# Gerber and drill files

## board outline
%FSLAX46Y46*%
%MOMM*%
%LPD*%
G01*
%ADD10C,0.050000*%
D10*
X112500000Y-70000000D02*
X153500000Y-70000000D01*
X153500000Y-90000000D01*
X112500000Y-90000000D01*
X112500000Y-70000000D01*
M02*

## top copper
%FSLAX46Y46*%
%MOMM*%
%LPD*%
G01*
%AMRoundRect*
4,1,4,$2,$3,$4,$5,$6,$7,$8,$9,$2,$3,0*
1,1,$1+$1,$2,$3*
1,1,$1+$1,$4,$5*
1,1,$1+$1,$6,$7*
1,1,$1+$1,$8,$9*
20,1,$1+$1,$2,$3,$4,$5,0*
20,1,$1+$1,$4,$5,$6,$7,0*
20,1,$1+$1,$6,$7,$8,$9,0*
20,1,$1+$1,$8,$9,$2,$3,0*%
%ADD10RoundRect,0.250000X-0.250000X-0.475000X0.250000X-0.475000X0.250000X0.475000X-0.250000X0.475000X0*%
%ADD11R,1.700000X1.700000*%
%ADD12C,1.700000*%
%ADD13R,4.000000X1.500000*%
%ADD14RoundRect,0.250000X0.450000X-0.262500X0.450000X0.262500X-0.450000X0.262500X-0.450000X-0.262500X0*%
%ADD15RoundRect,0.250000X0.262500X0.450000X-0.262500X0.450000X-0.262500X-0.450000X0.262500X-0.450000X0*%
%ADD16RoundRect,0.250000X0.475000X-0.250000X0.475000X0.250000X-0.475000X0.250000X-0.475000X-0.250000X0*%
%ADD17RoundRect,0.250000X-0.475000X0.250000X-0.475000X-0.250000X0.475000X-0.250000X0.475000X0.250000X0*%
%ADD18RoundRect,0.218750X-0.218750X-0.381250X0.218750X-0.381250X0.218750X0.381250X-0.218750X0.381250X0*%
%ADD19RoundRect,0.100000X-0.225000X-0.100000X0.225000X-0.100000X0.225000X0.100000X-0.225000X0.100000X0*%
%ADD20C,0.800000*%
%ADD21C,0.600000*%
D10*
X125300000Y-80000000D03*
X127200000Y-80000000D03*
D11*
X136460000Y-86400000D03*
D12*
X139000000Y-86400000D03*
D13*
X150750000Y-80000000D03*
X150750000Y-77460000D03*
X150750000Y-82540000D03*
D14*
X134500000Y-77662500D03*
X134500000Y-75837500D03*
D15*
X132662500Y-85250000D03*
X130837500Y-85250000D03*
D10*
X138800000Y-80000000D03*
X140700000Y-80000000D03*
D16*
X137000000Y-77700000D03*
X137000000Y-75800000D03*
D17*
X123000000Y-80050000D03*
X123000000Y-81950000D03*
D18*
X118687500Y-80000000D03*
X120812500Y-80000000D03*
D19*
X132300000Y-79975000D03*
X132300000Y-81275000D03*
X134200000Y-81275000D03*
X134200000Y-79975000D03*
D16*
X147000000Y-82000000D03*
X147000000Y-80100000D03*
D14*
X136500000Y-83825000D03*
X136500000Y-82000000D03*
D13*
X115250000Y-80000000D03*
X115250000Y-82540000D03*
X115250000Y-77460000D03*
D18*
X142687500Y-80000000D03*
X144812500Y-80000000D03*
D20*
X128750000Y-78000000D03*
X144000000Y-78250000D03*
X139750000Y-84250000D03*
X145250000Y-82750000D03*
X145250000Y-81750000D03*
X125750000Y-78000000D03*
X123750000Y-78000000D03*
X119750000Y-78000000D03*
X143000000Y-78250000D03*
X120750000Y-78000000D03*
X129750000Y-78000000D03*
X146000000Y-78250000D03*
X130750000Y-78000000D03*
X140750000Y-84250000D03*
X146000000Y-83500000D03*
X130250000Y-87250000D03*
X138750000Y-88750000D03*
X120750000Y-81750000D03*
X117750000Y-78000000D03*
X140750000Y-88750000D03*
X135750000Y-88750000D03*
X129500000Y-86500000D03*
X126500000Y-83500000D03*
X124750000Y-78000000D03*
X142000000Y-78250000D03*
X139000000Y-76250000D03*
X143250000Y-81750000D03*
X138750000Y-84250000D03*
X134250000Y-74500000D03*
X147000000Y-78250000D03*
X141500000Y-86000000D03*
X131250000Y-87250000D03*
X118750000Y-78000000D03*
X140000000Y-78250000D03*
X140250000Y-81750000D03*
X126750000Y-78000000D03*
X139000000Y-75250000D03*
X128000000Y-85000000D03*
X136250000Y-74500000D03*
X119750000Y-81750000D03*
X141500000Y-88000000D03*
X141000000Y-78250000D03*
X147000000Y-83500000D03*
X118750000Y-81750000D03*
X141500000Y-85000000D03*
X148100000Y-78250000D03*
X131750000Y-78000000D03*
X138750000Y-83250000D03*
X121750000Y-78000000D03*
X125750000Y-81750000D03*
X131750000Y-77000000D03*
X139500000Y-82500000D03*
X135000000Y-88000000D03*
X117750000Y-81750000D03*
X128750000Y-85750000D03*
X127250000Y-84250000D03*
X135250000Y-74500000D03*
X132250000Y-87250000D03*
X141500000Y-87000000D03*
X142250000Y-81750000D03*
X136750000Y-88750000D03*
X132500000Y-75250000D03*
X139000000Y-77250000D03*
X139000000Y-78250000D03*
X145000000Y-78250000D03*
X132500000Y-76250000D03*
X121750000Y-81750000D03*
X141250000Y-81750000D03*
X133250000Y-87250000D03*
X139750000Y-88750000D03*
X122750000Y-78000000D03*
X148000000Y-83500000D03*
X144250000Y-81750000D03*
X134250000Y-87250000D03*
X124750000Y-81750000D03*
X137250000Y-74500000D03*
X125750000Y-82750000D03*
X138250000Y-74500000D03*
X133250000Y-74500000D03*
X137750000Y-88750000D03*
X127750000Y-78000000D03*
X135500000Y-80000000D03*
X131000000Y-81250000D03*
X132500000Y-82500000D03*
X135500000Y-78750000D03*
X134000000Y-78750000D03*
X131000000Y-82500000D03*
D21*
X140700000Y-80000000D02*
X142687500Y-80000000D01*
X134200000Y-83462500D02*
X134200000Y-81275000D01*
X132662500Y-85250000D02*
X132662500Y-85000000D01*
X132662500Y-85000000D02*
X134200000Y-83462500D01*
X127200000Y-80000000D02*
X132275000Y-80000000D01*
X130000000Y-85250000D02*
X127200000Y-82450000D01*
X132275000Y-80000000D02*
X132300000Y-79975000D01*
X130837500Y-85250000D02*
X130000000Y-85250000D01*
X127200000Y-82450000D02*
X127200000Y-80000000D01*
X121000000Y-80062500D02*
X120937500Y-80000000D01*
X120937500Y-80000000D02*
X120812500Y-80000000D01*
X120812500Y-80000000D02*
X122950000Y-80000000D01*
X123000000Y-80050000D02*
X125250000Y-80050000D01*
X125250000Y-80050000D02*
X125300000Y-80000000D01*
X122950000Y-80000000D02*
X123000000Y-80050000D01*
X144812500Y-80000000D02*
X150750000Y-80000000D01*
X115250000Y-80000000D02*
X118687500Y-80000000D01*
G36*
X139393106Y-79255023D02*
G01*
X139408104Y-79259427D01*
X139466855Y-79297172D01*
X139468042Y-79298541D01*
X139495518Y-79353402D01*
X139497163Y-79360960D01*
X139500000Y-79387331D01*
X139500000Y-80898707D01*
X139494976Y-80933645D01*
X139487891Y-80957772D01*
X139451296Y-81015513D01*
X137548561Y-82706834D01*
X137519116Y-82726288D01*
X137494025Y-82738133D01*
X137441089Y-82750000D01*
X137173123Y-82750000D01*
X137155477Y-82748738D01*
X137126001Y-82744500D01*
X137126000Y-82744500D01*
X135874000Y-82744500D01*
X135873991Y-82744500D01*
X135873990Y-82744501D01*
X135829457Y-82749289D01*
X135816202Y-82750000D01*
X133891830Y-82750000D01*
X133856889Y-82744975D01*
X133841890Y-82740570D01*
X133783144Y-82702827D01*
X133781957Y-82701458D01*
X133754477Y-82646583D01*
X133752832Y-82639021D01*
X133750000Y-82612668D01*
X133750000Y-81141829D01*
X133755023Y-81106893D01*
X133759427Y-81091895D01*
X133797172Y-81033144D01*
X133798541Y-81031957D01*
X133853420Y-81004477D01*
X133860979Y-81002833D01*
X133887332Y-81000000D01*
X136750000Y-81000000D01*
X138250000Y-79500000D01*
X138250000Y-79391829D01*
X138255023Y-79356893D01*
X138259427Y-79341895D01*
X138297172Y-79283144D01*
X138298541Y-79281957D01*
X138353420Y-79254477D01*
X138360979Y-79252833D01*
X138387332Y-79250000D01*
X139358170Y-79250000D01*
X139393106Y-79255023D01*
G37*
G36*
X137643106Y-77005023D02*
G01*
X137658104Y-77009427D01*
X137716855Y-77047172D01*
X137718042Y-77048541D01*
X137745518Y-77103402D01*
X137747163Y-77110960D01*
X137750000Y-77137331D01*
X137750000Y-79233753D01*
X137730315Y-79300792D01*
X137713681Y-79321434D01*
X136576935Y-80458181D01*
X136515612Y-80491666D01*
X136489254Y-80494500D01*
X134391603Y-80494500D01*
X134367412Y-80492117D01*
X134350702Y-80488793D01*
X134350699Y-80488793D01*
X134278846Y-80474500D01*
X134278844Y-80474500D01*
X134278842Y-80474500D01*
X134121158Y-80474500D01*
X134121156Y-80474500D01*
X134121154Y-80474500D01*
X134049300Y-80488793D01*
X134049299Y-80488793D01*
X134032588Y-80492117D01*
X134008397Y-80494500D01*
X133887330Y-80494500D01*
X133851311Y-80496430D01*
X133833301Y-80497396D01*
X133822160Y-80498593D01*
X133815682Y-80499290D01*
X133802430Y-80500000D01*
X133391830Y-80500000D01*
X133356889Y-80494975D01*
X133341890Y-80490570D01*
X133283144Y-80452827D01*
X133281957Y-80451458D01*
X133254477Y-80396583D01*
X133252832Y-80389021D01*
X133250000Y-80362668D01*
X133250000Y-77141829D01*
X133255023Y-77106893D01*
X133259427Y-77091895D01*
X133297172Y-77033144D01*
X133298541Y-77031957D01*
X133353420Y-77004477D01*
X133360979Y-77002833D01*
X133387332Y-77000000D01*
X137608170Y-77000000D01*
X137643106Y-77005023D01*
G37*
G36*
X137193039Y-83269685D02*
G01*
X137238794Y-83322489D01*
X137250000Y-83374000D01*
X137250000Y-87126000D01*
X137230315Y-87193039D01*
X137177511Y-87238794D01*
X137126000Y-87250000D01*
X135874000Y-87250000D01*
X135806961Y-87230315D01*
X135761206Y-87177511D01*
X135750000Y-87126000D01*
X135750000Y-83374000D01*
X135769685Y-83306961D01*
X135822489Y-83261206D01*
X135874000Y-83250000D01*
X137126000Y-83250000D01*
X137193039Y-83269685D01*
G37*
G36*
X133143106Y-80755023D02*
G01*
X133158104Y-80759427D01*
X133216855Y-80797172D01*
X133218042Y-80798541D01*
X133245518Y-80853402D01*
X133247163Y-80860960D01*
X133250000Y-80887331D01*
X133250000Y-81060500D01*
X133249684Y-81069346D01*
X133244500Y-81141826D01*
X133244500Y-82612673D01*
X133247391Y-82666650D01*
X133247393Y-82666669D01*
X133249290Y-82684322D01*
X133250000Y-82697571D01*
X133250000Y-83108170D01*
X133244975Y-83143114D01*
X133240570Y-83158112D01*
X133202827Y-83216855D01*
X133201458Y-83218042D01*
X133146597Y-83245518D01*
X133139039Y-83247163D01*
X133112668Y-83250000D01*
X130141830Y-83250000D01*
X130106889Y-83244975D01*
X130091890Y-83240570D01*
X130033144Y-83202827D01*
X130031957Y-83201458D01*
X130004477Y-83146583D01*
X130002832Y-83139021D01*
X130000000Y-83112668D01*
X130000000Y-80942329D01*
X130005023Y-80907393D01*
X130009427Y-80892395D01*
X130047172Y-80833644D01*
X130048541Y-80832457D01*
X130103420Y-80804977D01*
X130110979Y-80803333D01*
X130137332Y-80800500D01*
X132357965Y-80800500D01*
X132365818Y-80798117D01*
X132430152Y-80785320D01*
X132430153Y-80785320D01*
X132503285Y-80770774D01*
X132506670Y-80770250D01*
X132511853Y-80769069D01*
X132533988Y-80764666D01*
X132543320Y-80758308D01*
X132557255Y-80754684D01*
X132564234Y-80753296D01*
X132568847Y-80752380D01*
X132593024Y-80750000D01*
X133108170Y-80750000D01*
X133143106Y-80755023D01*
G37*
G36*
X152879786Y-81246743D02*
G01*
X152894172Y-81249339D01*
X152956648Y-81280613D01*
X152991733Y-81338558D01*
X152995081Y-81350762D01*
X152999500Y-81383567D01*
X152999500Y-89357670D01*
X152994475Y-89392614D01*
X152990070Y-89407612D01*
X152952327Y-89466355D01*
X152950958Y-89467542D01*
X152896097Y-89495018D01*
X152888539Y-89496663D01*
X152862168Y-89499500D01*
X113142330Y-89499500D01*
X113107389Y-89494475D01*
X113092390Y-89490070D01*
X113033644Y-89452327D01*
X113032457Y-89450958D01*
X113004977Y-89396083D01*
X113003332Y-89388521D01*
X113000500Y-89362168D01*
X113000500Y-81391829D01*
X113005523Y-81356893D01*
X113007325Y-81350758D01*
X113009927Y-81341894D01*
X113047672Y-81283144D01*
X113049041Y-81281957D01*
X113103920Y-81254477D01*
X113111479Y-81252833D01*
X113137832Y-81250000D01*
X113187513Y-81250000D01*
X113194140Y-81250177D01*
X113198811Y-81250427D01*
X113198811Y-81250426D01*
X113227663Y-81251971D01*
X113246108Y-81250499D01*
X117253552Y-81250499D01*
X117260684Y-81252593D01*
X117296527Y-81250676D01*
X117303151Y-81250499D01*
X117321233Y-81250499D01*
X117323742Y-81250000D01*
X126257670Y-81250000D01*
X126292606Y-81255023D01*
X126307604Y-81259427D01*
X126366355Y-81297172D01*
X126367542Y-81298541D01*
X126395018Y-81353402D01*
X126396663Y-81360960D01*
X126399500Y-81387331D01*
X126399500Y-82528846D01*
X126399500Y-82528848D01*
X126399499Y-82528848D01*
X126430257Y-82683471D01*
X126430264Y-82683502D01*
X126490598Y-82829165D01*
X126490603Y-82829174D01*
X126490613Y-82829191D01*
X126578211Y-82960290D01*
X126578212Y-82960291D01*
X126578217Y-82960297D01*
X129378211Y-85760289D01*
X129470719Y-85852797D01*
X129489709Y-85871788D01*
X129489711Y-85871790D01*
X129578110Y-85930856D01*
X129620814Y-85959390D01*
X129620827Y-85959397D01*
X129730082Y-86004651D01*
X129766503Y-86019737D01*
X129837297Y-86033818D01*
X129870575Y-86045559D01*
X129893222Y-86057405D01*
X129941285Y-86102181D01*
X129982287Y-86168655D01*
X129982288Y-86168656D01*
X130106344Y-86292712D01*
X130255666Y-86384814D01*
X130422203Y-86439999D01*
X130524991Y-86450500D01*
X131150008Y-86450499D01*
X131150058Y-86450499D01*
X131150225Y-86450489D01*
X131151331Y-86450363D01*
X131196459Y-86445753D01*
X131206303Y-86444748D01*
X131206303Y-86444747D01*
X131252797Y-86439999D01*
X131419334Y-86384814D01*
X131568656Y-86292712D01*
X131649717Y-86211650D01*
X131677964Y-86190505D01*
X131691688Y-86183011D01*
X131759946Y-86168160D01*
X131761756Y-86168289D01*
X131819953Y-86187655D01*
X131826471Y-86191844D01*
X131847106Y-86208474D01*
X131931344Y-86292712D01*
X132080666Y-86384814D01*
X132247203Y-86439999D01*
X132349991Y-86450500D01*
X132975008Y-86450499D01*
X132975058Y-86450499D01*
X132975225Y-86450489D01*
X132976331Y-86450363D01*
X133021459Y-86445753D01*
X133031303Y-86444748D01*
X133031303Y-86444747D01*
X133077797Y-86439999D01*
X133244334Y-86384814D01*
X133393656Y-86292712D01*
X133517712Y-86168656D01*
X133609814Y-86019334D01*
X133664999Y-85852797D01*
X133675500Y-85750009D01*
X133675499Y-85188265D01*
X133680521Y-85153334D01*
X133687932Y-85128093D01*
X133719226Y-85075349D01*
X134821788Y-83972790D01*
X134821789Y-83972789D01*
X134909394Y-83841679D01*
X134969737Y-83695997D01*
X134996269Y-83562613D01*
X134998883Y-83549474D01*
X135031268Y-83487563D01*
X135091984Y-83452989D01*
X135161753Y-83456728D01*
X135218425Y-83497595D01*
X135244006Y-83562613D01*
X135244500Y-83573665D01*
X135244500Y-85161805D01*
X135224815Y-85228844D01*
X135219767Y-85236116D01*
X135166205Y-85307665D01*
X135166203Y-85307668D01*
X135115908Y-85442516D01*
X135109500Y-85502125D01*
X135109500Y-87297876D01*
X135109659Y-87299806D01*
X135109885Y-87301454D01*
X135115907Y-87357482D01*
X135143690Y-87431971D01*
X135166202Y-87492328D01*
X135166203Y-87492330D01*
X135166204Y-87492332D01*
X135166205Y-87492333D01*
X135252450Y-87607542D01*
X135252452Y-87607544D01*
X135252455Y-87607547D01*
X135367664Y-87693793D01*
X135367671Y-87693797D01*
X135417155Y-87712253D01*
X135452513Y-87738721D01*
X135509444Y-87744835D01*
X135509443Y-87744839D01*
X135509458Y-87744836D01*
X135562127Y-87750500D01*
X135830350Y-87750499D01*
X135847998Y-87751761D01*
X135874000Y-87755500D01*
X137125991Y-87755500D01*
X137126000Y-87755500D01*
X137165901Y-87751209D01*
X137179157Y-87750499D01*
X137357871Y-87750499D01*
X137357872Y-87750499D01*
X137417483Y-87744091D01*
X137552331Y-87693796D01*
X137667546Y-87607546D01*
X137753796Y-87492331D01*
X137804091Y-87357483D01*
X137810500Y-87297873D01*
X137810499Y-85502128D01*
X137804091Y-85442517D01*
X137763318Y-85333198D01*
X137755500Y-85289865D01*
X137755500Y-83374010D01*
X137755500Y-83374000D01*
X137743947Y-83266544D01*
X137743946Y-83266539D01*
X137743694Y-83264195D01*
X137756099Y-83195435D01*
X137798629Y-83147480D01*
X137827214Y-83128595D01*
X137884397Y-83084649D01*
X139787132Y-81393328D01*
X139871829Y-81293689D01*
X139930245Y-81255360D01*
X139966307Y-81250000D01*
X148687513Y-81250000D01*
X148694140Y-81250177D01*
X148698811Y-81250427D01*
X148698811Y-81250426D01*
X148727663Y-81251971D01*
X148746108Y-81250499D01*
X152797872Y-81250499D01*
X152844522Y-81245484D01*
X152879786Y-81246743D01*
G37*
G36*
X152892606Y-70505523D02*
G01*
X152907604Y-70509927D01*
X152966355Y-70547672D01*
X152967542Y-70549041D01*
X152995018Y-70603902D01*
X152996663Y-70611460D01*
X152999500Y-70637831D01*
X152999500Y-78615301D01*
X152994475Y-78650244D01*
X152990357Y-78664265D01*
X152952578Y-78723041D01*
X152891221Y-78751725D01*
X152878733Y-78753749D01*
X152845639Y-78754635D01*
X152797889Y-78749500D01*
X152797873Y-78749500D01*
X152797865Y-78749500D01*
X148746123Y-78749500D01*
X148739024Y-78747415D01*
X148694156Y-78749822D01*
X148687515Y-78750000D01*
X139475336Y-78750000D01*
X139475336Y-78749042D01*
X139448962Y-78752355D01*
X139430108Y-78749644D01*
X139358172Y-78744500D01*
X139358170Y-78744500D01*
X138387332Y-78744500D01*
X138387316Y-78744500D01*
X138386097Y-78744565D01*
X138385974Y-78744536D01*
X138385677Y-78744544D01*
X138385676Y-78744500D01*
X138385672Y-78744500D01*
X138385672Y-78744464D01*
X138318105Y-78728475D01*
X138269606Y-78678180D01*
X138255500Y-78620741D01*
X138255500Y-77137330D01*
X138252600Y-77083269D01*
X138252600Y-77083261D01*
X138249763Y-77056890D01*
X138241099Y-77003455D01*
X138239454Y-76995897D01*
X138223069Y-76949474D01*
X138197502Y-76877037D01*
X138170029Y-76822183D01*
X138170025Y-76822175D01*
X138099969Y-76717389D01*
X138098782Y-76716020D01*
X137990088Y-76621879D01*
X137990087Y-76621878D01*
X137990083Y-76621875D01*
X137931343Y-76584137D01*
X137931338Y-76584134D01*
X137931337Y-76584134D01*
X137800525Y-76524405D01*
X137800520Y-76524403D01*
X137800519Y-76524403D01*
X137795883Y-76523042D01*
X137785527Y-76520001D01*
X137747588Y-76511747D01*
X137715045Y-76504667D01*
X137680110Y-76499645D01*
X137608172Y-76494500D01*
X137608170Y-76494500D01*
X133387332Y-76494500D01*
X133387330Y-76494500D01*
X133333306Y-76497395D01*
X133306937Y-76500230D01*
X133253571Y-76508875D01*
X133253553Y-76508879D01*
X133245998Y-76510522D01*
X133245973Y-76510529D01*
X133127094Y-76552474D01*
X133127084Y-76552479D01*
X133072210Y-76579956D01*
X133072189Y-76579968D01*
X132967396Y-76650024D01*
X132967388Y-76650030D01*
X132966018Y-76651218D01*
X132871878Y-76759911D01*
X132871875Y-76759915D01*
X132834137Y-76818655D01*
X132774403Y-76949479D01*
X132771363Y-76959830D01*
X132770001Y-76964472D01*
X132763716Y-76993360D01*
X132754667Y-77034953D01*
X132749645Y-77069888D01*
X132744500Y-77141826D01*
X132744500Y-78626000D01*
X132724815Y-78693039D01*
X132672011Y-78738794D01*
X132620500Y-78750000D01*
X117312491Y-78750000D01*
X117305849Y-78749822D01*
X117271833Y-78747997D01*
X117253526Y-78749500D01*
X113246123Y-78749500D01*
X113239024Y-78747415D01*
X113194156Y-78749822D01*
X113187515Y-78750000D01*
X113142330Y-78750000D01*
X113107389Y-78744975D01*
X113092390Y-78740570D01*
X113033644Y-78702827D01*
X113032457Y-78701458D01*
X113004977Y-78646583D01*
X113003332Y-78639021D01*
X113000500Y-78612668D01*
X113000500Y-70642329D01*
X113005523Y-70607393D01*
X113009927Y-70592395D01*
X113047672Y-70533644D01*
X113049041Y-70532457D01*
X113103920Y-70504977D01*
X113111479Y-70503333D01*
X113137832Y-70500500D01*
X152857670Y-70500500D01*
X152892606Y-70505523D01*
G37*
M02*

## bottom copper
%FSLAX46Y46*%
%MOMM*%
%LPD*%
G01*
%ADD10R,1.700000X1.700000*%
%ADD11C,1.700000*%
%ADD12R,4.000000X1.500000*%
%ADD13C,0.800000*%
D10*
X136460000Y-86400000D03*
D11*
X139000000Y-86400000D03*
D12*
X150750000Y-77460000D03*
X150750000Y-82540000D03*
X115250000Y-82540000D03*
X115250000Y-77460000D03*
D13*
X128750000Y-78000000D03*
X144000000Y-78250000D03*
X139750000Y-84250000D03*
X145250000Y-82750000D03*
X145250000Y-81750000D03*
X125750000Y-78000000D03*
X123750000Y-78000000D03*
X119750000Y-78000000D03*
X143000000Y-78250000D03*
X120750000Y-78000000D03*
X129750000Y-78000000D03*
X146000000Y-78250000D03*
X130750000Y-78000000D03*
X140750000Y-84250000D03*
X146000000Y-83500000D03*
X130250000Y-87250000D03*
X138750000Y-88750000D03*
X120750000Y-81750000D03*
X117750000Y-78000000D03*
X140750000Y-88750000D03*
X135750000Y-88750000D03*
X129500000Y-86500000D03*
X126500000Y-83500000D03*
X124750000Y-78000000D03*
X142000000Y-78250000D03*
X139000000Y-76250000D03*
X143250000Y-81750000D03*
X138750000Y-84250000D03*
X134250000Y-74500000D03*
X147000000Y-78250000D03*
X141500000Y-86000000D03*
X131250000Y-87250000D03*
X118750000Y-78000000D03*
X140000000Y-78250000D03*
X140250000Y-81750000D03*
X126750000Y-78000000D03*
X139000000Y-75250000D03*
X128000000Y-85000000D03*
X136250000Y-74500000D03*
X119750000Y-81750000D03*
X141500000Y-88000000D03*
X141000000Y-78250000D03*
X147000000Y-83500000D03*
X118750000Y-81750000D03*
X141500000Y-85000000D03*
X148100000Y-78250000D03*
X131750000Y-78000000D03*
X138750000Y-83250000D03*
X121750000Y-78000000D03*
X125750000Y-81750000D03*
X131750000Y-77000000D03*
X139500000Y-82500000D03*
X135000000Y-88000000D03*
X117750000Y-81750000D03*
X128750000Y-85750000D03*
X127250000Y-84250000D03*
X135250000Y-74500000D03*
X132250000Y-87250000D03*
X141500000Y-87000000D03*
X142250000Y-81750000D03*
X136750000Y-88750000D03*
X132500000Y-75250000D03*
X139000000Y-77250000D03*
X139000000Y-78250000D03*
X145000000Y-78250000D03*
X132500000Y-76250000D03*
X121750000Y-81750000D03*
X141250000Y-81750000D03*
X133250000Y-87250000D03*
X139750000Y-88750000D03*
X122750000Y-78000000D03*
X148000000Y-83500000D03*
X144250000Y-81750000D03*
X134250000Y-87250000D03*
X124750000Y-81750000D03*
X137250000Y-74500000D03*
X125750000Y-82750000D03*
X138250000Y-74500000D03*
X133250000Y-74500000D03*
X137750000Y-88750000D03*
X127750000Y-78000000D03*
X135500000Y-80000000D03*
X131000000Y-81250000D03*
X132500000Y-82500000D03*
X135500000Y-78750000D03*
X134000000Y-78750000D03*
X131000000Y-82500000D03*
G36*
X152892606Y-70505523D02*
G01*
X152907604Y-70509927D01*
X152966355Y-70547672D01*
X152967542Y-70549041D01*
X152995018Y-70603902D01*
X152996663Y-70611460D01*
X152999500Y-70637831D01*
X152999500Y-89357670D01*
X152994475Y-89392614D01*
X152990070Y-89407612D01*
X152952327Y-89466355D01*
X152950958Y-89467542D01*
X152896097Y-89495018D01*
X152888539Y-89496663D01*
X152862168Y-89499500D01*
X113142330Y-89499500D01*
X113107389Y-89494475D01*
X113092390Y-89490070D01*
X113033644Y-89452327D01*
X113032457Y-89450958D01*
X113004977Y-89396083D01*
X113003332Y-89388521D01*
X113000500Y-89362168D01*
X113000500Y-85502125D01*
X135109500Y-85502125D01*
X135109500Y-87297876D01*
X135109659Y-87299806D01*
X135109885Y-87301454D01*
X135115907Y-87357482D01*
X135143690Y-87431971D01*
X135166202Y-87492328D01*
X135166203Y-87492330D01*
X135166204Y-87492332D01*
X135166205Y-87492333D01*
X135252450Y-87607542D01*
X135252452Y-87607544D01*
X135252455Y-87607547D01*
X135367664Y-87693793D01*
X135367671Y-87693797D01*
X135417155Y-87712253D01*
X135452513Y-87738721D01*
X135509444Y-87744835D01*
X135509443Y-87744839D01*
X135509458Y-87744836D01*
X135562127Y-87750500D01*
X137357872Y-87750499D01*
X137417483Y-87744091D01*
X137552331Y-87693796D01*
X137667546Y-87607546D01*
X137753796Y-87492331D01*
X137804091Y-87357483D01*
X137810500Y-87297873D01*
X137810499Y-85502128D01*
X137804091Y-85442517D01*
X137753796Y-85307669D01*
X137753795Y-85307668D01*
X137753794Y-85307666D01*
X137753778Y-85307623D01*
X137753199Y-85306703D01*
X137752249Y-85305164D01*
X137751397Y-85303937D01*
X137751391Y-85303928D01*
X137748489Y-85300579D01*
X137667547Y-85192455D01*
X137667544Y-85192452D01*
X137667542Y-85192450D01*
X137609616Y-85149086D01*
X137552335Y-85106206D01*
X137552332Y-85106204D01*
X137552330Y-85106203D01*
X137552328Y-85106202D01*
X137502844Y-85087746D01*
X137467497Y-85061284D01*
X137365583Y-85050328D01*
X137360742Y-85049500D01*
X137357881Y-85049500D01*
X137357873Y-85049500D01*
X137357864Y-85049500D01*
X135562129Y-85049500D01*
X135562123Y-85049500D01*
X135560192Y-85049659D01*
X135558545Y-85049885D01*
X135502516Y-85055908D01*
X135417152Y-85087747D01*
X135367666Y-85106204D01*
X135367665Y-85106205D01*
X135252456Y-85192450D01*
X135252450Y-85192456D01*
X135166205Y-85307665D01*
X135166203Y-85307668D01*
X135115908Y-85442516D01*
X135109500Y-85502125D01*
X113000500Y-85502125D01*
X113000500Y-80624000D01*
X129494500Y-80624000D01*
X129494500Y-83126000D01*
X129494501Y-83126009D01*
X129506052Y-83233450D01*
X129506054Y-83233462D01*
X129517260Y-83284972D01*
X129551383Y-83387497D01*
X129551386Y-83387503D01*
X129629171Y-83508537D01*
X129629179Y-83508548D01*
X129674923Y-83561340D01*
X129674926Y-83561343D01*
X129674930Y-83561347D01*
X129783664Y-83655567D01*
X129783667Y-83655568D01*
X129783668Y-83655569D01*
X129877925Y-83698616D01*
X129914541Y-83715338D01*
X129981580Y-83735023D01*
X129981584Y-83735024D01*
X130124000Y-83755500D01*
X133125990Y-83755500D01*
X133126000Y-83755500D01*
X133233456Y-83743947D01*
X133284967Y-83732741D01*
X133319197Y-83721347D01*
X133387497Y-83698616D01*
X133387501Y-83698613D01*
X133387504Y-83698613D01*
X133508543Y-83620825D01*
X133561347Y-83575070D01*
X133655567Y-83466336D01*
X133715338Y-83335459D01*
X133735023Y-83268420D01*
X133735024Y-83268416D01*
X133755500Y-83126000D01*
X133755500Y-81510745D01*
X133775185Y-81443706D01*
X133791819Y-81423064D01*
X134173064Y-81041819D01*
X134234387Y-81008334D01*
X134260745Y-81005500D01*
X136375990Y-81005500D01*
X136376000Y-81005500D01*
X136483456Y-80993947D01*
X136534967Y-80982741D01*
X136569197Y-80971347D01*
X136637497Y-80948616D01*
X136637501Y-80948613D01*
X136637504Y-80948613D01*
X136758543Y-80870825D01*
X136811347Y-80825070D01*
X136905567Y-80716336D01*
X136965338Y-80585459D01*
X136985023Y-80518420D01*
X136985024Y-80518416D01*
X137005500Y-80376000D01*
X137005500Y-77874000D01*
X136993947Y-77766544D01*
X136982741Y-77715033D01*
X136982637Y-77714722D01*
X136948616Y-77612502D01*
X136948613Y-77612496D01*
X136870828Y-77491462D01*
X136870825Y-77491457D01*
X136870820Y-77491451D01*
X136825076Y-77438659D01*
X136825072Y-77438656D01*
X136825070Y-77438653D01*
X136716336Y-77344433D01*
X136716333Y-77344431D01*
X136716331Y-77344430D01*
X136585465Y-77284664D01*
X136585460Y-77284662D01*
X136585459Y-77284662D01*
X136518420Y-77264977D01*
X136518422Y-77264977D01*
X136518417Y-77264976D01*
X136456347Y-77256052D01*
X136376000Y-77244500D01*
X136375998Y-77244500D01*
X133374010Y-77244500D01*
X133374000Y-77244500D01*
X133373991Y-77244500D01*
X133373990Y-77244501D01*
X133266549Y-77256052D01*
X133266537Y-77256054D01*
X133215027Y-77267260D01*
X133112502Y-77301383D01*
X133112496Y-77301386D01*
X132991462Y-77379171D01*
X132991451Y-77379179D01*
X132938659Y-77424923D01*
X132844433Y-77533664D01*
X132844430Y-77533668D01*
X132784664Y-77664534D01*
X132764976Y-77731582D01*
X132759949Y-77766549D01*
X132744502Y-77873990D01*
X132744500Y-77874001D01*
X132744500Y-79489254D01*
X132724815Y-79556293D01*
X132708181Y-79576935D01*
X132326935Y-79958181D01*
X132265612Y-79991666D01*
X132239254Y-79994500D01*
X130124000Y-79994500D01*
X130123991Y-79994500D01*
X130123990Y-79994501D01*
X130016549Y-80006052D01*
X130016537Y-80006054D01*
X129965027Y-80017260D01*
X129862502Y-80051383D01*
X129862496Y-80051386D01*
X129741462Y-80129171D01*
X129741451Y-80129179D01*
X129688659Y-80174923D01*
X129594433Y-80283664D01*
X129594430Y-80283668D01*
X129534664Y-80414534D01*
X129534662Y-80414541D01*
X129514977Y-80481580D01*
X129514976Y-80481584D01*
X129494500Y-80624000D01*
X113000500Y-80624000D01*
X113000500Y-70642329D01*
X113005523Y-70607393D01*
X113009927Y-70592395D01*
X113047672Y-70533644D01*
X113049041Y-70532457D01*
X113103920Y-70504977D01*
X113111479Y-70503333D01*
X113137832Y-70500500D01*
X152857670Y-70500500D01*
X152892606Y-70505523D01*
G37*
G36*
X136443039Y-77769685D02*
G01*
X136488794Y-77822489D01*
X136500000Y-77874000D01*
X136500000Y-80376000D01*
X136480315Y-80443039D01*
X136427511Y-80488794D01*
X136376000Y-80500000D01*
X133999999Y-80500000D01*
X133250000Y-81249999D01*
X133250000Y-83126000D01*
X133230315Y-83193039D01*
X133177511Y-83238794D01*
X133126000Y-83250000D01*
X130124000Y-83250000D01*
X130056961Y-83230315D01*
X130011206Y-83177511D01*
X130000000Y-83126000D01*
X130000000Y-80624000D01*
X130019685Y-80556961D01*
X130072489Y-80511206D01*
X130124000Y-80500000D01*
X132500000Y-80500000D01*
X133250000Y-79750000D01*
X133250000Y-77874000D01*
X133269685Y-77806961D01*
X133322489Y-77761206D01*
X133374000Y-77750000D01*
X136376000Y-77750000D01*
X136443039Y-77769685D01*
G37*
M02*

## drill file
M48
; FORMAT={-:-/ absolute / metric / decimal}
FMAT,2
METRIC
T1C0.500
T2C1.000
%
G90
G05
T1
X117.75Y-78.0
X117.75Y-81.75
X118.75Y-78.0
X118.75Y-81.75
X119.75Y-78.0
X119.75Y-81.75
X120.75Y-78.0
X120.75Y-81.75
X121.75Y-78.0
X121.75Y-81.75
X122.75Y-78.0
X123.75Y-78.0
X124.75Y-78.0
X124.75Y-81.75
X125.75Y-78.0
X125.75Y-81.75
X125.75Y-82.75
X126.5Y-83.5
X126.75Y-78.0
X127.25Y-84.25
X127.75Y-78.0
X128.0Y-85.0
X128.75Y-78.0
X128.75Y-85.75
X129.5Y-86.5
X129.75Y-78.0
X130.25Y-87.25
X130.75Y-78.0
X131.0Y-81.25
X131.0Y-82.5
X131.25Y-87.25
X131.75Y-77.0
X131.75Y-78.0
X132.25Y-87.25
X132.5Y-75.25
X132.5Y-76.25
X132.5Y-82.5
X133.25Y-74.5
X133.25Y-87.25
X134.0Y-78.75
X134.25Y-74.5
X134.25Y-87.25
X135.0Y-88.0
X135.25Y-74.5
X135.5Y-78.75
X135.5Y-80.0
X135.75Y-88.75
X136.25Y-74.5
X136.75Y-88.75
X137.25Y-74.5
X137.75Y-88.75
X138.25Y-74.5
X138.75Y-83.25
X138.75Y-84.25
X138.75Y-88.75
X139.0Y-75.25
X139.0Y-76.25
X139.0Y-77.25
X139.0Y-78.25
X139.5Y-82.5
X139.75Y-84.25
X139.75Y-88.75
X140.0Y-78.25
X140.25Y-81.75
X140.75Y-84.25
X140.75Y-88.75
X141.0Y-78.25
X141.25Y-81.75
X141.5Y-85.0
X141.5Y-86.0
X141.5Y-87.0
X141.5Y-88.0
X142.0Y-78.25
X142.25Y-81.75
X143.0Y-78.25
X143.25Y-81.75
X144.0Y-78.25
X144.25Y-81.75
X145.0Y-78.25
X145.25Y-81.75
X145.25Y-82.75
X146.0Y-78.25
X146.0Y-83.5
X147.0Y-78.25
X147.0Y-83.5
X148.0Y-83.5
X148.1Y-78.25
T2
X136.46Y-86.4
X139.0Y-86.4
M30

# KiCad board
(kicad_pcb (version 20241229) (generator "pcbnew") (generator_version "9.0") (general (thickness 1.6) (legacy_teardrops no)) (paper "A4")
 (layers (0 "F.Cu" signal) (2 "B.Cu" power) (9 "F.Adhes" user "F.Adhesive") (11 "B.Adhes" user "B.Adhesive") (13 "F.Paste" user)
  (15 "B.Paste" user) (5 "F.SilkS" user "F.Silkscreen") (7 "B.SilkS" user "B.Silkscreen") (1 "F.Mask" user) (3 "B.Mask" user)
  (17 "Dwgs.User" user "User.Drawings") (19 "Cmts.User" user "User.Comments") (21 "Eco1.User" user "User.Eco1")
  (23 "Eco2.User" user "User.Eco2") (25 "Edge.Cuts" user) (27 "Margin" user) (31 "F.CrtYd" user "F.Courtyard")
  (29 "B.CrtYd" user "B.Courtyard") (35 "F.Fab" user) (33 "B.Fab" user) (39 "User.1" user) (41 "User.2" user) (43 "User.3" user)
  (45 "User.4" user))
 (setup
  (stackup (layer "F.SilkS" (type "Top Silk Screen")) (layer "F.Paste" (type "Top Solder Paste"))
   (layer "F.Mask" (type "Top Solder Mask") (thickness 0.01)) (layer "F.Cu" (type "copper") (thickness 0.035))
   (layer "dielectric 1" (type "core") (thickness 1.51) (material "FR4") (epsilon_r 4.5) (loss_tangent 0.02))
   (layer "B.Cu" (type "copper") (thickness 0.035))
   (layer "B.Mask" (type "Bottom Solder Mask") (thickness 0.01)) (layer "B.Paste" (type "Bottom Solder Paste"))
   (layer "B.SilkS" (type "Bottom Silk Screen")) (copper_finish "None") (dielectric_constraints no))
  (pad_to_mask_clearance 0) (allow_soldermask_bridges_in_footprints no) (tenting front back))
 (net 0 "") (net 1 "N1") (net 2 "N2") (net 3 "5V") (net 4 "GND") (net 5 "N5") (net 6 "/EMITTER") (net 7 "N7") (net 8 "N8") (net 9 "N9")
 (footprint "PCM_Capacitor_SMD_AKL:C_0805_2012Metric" (layer "F.Cu") (at 126.25 80)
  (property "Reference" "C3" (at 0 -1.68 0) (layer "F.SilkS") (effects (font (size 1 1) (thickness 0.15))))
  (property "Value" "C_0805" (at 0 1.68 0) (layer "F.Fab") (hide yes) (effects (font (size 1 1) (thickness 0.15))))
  (pad "1" smd roundrect (at -0.95 0) (size 1 1.45) (layers "F.Cu" "F.Mask" "F.Paste") (roundrect_rratio 0.25) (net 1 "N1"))
  (pad "2" smd roundrect (at 0.95 0) (size 1 1.45) (layers "F.Cu" "F.Mask" "F.Paste") (roundrect_rratio 0.25) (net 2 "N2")))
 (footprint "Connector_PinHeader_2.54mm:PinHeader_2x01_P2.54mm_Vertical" (layer "F.Cu") (at 136.46 86.4)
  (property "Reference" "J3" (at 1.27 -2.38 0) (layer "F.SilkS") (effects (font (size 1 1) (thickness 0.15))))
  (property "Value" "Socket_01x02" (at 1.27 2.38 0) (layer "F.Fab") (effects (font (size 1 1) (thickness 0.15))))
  (pad "1" thru_hole rect (at 0 0) (size 1.7 1.7) (drill 1) (layers "*.Cu" "*.Mask") (remove_unused_layers no) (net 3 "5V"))
  (pad "2" thru_hole circle (at 2.54 0) (size 1.7 1.7) (drill 1) (layers "*.Cu" "*.Mask") (remove_unused_layers no) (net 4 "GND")))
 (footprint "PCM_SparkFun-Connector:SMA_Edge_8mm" (layer "F.Cu") (at 150.75 80 -90)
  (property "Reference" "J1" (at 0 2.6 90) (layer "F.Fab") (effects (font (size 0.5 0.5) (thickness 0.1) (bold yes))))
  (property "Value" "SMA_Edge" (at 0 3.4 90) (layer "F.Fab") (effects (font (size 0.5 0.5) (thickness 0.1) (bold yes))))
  (pad "1" smd rect (at 0 0 270) (size 1.5 4) (layers "F.Cu" "F.Mask") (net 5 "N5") (thermal_bridge_angle 0))
  (pad "2" smd rect (at -2.54 0 270) (size 1.5 4) (layers "F.Cu" "F.Mask") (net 4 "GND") (thermal_bridge_angle 0))
  (pad "2" smd rect (at -2.54 0 270) (size 1.5 4) (layers "B.Cu" "B.Mask") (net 4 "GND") (thermal_bridge_angle 0))
  (pad "2" smd rect (at 2.54 0 270) (size 1.5 4) (layers "F.Cu" "F.Mask") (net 4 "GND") (thermal_bridge_angle 0))
  (pad "2" smd rect (at 2.54 0 270) (size 1.5 4) (layers "B.Cu" "B.Mask") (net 4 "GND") (thermal_bridge_angle 0)))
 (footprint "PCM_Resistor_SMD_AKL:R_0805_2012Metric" (layer "F.Cu") (at 134.5 76.75 90)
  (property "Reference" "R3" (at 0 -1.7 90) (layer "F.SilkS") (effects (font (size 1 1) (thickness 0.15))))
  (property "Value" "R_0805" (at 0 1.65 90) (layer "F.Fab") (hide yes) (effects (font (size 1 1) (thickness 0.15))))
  (pad "1" smd roundrect (at -0.9125 0 90) (size 1.025 1.4) (layers "F.Cu" "F.Mask" "F.Paste") (roundrect_rratio 0.243902)
   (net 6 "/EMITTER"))
  (pad "2" smd roundrect (at 0.9125 0 90) (size 1.025 1.4) (layers "F.Cu" "F.Mask" "F.Paste") (roundrect_rratio 0.243902) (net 4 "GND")))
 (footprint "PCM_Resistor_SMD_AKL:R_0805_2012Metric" (layer "F.Cu") (at 131.75 85.25 180)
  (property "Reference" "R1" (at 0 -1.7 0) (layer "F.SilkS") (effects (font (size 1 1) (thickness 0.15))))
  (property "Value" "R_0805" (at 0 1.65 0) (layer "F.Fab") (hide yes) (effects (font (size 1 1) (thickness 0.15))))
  (pad "1" smd roundrect (at -0.9125 0 180) (size 1.025 1.4) (layers "F.Cu" "F.Mask" "F.Paste") (roundrect_rratio 0.243902) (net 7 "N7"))
  (pad "2" smd roundrect (at 0.9125 0 180) (size 1.025 1.4) (layers "F.Cu" "F.Mask" "F.Paste") (roundrect_rratio 0.243902) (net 2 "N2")))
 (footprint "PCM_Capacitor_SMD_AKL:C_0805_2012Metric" (layer "F.Cu") (at 139.75 80)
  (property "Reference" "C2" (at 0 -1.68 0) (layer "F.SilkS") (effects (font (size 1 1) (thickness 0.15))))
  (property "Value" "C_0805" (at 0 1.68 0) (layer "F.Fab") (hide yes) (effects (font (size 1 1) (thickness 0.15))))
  (pad "1" smd roundrect (at -0.95 0) (size 1 1.45) (layers "F.Cu" "F.Mask" "F.Paste") (roundrect_rratio 0.25) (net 7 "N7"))
  (pad "2" smd roundrect (at 0.95 0) (size 1 1.45) (layers "F.Cu" "F.Mask" "F.Paste") (roundrect_rratio 0.25) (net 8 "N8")))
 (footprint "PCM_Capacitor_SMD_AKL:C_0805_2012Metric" (layer "F.Cu") (at 137 76.75 90)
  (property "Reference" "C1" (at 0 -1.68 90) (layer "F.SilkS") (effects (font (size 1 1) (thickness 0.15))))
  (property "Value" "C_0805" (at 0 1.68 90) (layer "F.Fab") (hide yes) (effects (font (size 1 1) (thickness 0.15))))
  (pad "1" smd roundrect (at -0.95 0 90) (size 1 1.45) (layers "F.Cu" "F.Mask" "F.Paste") (roundrect_rratio 0.25) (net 6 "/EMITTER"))
  (pad "2" smd roundrect (at 0.95 0 90) (size 1 1.45) (layers "F.Cu" "F.Mask" "F.Paste") (roundrect_rratio 0.25) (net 4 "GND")))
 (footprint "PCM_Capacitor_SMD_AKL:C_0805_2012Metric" (layer "F.Cu") (at 123 81 -90)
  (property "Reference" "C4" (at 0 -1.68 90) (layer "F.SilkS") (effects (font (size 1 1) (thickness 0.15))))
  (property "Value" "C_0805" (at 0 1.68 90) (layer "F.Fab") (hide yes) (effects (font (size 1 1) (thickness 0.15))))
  (pad "1" smd roundrect (at -0.95 0 270) (size 1 1.45) (layers "F.Cu" "F.Mask" "F.Paste") (roundrect_rratio 0.25) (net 1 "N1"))
  (pad "2" smd roundrect (at 0.95 0 270) (size 1 1.45) (layers "F.Cu" "F.Mask" "F.Paste") (roundrect_rratio 0.25) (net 4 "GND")))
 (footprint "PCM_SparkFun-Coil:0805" (layer "F.Cu") (at 119.75 80)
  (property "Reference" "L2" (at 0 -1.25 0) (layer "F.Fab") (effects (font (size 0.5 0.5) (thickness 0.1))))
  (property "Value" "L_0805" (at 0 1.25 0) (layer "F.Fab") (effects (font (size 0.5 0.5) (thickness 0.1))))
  (pad "1" smd roundrect (at -1.0625 0) (size 0.875 1.2) (layers "F.Cu" "F.Mask" "F.Paste") (roundrect_rratio 0.25) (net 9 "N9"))
  (pad "2" smd roundrect (at 1.0625 0) (size 0.875 1.2) (layers "F.Cu" "F.Mask" "F.Paste") (roundrect_rratio 0.25) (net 1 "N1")))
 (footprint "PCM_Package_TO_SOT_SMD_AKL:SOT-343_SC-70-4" (layer "F.Cu") (at 133.25 80.625)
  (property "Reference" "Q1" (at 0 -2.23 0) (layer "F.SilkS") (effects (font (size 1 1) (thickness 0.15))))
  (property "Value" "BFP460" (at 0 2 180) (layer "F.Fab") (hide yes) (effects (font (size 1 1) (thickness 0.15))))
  (pad "1" smd roundrect (at -0.95 -0.65) (size 0.65 0.4) (layers "F.Cu" "F.Mask" "F.Paste") (roundrect_rratio 0.25) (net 2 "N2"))
  (pad "2" smd roundrect (at -0.95 0.65) (size 0.65 0.4) (layers "F.Cu" "F.Mask" "F.Paste") (roundrect_rratio 0.25) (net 6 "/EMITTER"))
  (pad "3" smd roundrect (at 0.95 0.65) (size 0.65 0.4) (layers "F.Cu" "F.Mask" "F.Paste") (roundrect_rratio 0.25) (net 7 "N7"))
  (pad "4" smd roundrect (at 0.95 -0.65) (size 0.65 0.4) (layers "F.Cu" "F.Mask" "F.Paste") (roundrect_rratio 0.25) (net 6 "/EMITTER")))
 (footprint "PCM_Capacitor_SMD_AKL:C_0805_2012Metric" (layer "F.Cu") (at 147 81.05 90)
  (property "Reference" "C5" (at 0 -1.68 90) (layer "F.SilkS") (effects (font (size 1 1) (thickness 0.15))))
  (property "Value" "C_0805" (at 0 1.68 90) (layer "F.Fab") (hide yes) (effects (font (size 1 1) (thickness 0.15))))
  (pad "1" smd roundrect (at -0.95 0 90) (size 1 1.45) (layers "F.Cu" "F.Mask" "F.Paste") (roundrect_rratio 0.25) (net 4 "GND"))
  (pad "2" smd roundrect (at 0.95 0 90) (size 1 1.45) (layers "F.Cu" "F.Mask" "F.Paste") (roundrect_rratio 0.25) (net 5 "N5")))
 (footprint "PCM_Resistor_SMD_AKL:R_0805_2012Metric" (layer "F.Cu") (at 136.5 82.9125 90)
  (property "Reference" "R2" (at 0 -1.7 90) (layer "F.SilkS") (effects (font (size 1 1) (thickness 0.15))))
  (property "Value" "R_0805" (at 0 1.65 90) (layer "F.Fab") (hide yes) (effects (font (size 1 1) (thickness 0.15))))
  (pad "1" smd roundrect (at -0.9125 0 90) (size 1.025 1.4) (layers "F.Cu" "F.Mask" "F.Paste") (roundrect_rratio 0.243902) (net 3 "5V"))
  (pad "2" smd roundrect (at 0.9125 0 90) (size 1.025 1.4) (layers "F.Cu" "F.Mask" "F.Paste") (roundrect_rratio 0.243902) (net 7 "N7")))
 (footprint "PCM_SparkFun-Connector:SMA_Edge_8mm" (layer "F.Cu") (at 115.25 80 90)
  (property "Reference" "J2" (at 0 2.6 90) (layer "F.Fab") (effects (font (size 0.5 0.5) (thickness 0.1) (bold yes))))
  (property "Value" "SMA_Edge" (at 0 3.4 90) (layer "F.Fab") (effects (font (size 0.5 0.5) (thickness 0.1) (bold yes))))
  (pad "1" smd rect (at 0 0 90) (size 1.5 4) (layers "F.Cu" "F.Mask") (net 9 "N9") (thermal_bridge_angle 0))
  (pad "2" smd rect (at -2.54 0 90) (size 1.5 4) (layers "F.Cu" "F.Mask") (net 4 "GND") (thermal_bridge_angle 0))
  (pad "2" smd rect (at -2.54 0 90) (size 1.5 4) (layers "B.Cu" "B.Mask") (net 4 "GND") (thermal_bridge_angle 0))
  (pad "2" smd rect (at 2.54 0 90) (size 1.5 4) (layers "F.Cu" "F.Mask") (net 4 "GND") (thermal_bridge_angle 0))
  (pad "2" smd rect (at 2.54 0 90) (size 1.5 4) (layers "B.Cu" "B.Mask") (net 4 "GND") (thermal_bridge_angle 0)))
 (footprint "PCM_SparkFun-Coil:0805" (layer "F.Cu") (at 143.75 80)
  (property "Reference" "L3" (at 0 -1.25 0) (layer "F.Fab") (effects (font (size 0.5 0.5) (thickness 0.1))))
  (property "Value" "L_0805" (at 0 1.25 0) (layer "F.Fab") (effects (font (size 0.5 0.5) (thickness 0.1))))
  (pad "1" smd roundrect (at -1.0625 0) (size 0.875 1.2) (layers "F.Cu" "F.Mask" "F.Paste") (roundrect_rratio 0.25) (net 8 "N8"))
  (pad "2" smd roundrect (at 1.0625 0) (size 0.875 1.2) (layers "F.Cu" "F.Mask" "F.Paste") (roundrect_rratio 0.25) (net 5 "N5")))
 (gr_rect (start 112.5 70) (end 153.5 90) (stroke (width 0.05) (type default)) (fill no) (layer "Edge.Cuts"))
 (via (at 128.75 78) (size 0.8) (drill 0.5) (layers "F.Cu" "B.Cu") (free yes) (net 4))
 (via (at 144 78.25) (size 0.8) (drill 0.5) (layers "F.Cu" "B.Cu") (free yes) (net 4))
 (via (at 139.75 84.25) (size 0.8) (drill 0.5) (layers "F.Cu" "B.Cu") (free yes) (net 4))
 (via (at 145.25 82.75) (size 0.8) (drill 0.5) (layers "F.Cu" "B.Cu") (free yes) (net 4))
 (via (at 145.25 81.75) (size 0.8) (drill 0.5) (layers "F.Cu" "B.Cu") (free yes) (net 4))
 (via (at 125.75 78) (size 0.8) (drill 0.5) (layers "F.Cu" "B.Cu") (free yes) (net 4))
 (via (at 123.75 78) (size 0.8) (drill 0.5) (layers "F.Cu" "B.Cu") (free yes) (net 4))
 (via (at 119.75 78) (size 0.8) (drill 0.5) (layers "F.Cu" "B.Cu") (free yes) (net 4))
 (via (at 143 78.25) (size 0.8) (drill 0.5) (layers "F.Cu" "B.Cu") (free yes) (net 4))
 (via (at 120.75 78) (size 0.8) (drill 0.5) (layers "F.Cu" "B.Cu") (free yes) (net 4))
 (via (at 129.75 78) (size 0.8) (drill 0.5) (layers "F.Cu" "B.Cu") (free yes) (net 4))
 (via (at 146 78.25) (size 0.8) (drill 0.5) (layers "F.Cu" "B.Cu") (free yes) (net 4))
 (via (at 130.75 78) (size 0.8) (drill 0.5) (layers "F.Cu" "B.Cu") (free yes) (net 4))
 (via (at 140.75 84.25) (size 0.8) (drill 0.5) (layers "F.Cu" "B.Cu") (free yes) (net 4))
 (via (at 146 83.5) (size 0.8) (drill 0.5) (layers "F.Cu" "B.Cu") (free yes) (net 4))
 (via (at 130.25 87.25) (size 0.8) (drill 0.5) (layers "F.Cu" "B.Cu") (free yes) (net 4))
 (via (at 138.75 88.75) (size 0.8) (drill 0.5) (layers "F.Cu" "B.Cu") (free yes) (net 4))
 (via (at 120.75 81.75) (size 0.8) (drill 0.5) (layers "F.Cu" "B.Cu") (free yes) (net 4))
 (via (at 117.75 78) (size 0.8) (drill 0.5) (layers "F.Cu" "B.Cu") (free yes) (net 4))
 (via (at 140.75 88.75) (size 0.8) (drill 0.5) (layers "F.Cu" "B.Cu") (free yes) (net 4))
 (via (at 135.75 88.75) (size 0.8) (drill 0.5) (layers "F.Cu" "B.Cu") (free yes) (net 4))
 (via (at 129.5 86.5) (size 0.8) (drill 0.5) (layers "F.Cu" "B.Cu") (free yes) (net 4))
 (via (at 126.5 83.5) (size 0.8) (drill 0.5) (layers "F.Cu" "B.Cu") (free yes) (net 4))
 (via (at 124.75 78) (size 0.8) (drill 0.5) (layers "F.Cu" "B.Cu") (free yes) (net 4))
 (via (at 142 78.25) (size 0.8) (drill 0.5) (layers "F.Cu" "B.Cu") (free yes) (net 4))
 (via (at 139 76.25) (size 0.8) (drill 0.5) (layers "F.Cu" "B.Cu") (free yes) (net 4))
 (via (at 143.25 81.75) (size 0.8) (drill 0.5) (layers "F.Cu" "B.Cu") (free yes) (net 4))
 (via (at 138.75 84.25) (size 0.8) (drill 0.5) (layers "F.Cu" "B.Cu") (free yes) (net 4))
 (via (at 134.25 74.5) (size 0.8) (drill 0.5) (layers "F.Cu" "B.Cu") (free yes) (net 4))
 (via (at 147 78.25) (size 0.8) (drill 0.5) (layers "F.Cu" "B.Cu") (free yes) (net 4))
 (via (at 141.5 86) (size 0.8) (drill 0.5) (layers "F.Cu" "B.Cu") (free yes) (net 4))
 (via (at 131.25 87.25) (size 0.8) (drill 0.5) (layers "F.Cu" "B.Cu") (free yes) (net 4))
 (via (at 118.75 78) (size 0.8) (drill 0.5) (layers "F.Cu" "B.Cu") (free yes) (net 4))
 (via (at 140 78.25) (size 0.8) (drill 0.5) (layers "F.Cu" "B.Cu") (free yes) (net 4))
 (via (at 140.25 81.75) (size 0.8) (drill 0.5) (layers "F.Cu" "B.Cu") (free yes) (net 4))
 (via (at 126.75 78) (size 0.8) (drill 0.5) (layers "F.Cu" "B.Cu") (free yes) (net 4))
 (via (at 139 75.25) (size 0.8) (drill 0.5) (layers "F.Cu" "B.Cu") (free yes) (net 4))
 (via (at 128 85) (size 0.8) (drill 0.5) (layers "F.Cu" "B.Cu") (free yes) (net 4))
 (via (at 136.25 74.5) (size 0.8) (drill 0.5) (layers "F.Cu" "B.Cu") (free yes) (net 4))
 (via (at 119.75 81.75) (size 0.8) (drill 0.5) (layers "F.Cu" "B.Cu") (free yes) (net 4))
 (via (at 141.5 88) (size 0.8) (drill 0.5) (layers "F.Cu" "B.Cu") (free yes) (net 4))
 (via (at 141 78.25) (size 0.8) (drill 0.5) (layers "F.Cu" "B.Cu") (free yes) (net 4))
 (via (at 147 83.5) (size 0.8) (drill 0.5) (layers "F.Cu" "B.Cu") (free yes) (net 4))
 (via (at 118.75 81.75) (size 0.8) (drill 0.5) (layers "F.Cu" "B.Cu") (free yes) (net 4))
 (via (at 141.5 85) (size 0.8) (drill 0.5) (layers "F.Cu" "B.Cu") (free yes) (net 4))
 (via (at 148.1 78.25) (size 0.8) (drill 0.5) (layers "F.Cu" "B.Cu") (free yes) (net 4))
 (via (at 131.75 78) (size 0.8) (drill 0.5) (layers "F.Cu" "B.Cu") (free yes) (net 4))
 (via (at 138.75 83.25) (size 0.8) (drill 0.5) (layers "F.Cu" "B.Cu") (free yes) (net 4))
 (via (at 121.75 78) (size 0.8) (drill 0.5) (layers "F.Cu" "B.Cu") (free yes) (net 4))
 (via (at 125.75 81.75) (size 0.8) (drill 0.5) (layers "F.Cu" "B.Cu") (free yes) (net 4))
 (via (at 131.75 77) (size 0.8) (drill 0.5) (layers "F.Cu" "B.Cu") (free yes) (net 4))
 (via (at 139.5 82.5) (size 0.8) (drill 0.5) (layers "F.Cu" "B.Cu") (free yes) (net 4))
 (via (at 135 88) (size 0.8) (drill 0.5) (layers "F.Cu" "B.Cu") (free yes) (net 4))
 (via (at 117.75 81.75) (size 0.8) (drill 0.5) (layers "F.Cu" "B.Cu") (free yes) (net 4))
 (via (at 128.75 85.75) (size 0.8) (drill 0.5) (layers "F.Cu" "B.Cu") (free yes) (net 4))
 (via (at 127.25 84.25) (size 0.8) (drill 0.5) (layers "F.Cu" "B.Cu") (free yes) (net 4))
 (via (at 135.25 74.5) (size 0.8) (drill 0.5) (layers "F.Cu" "B.Cu") (free yes) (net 4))
 (via (at 132.25 87.25) (size 0.8) (drill 0.5) (layers "F.Cu" "B.Cu") (free yes) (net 4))
 (via (at 141.5 87) (size 0.8) (drill 0.5) (layers "F.Cu" "B.Cu") (free yes) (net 4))
 (via (at 142.25 81.75) (size 0.8) (drill 0.5) (layers "F.Cu" "B.Cu") (free yes) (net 4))
 (via (at 136.75 88.75) (size 0.8) (drill 0.5) (layers "F.Cu" "B.Cu") (free yes) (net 4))
 (via (at 132.5 75.25) (size 0.8) (drill 0.5) (layers "F.Cu" "B.Cu") (free yes) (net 4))
 (via (at 139 77.25) (size 0.8) (drill 0.5) (layers "F.Cu" "B.Cu") (free yes) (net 4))
 (via (at 139 78.25) (size 0.8) (drill 0.5) (layers "F.Cu" "B.Cu") (free yes) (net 4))
 (via (at 145 78.25) (size 0.8) (drill 0.5) (layers "F.Cu" "B.Cu") (free yes) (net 4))
 (via (at 132.5 76.25) (size 0.8) (drill 0.5) (layers "F.Cu" "B.Cu") (free yes) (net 4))
 (via (at 121.75 81.75) (size 0.8) (drill 0.5) (layers "F.Cu" "B.Cu") (free yes) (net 4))
 (via (at 141.25 81.75) (size 0.8) (drill 0.5) (layers "F.Cu" "B.Cu") (free yes) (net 4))
 (via (at 133.25 87.25) (size 0.8) (drill 0.5) (layers "F.Cu" "B.Cu") (free yes) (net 4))
 (via (at 139.75 88.75) (size 0.8) (drill 0.5) (layers "F.Cu" "B.Cu") (free yes) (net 4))
 (via (at 122.75 78) (size 0.8) (drill 0.5) (layers "F.Cu" "B.Cu") (free yes) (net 4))
 (via (at 148 83.5) (size 0.8) (drill 0.5) (layers "F.Cu" "B.Cu") (free yes) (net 4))
 (via (at 144.25 81.75) (size 0.8) (drill 0.5) (layers "F.Cu" "B.Cu") (free yes) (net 4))
 (via (at 134.25 87.25) (size 0.8) (drill 0.5) (layers "F.Cu" "B.Cu") (free yes) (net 4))
 (via (at 124.75 81.75) (size 0.8) (drill 0.5) (layers "F.Cu" "B.Cu") (free yes) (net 4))
 (via (at 137.25 74.5) (size 0.8) (drill 0.5) (layers "F.Cu" "B.Cu") (free yes) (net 4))
 (via (at 125.75 82.75) (size 0.8) (drill 0.5) (layers "F.Cu" "B.Cu") (free yes) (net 4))
 (via (at 138.25 74.5) (size 0.8) (drill 0.5) (layers "F.Cu" "B.Cu") (free yes) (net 4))
 (via (at 133.25 74.5) (size 0.8) (drill 0.5) (layers "F.Cu" "B.Cu") (free yes) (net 4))
 (via (at 137.75 88.75) (size 0.8) (drill 0.5) (layers "F.Cu" "B.Cu") (free yes) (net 4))
 (via (at 127.75 78) (size 0.8) (drill 0.5) (layers "F.Cu" "B.Cu") (free yes) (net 4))
 (via (at 135.5 80) (size 0.8) (drill 0.5) (layers "F.Cu" "B.Cu") (free yes) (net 6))
 (via (at 131 81.25) (size 0.8) (drill 0.5) (layers "F.Cu" "B.Cu") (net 6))
 (via (at 132.5 82.5) (size 0.8) (drill 0.5) (layers "F.Cu" "B.Cu") (free yes) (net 6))
 (via (at 135.5 78.75) (size 0.8) (drill 0.5) (layers "F.Cu" "B.Cu") (free yes) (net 6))
 (via (at 134 78.75) (size 0.8) (drill 0.5) (layers "F.Cu" "B.Cu") (free yes) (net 6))
 (via (at 131 82.5) (size 0.8) (drill 0.5) (layers "F.Cu" "B.Cu") (free yes) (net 6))
 (segment (start 140.7 80) (end 142.6875 80) (width 0.6) (layer "F.Cu") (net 8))
 (segment (start 134.2 83.4625) (end 134.2 81.275) (width 0.6) (layer "F.Cu") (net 7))
 (segment (start 132.6625 85.25) (end 132.6625 85) (width 0.6) (layer "F.Cu") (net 7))
 (segment (start 132.6625 85) (end 134.2 83.4625) (width 0.6) (layer "F.Cu") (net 7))
 (segment (start 127.2 80) (end 132.275 80) (width 0.6) (layer "F.Cu") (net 2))
 (segment (start 130 85.25) (end 127.2 82.45) (width 0.6) (layer "F.Cu") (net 2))
 (segment (start 132.275 80) (end 132.3 79.975) (width 0.6) (layer "F.Cu") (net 2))
 (segment (start 130.8375 85.25) (end 130 85.25) (width 0.6) (layer "F.Cu") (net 2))
 (segment (start 127.2 82.45) (end 127.2 80) (width 0.6) (layer "F.Cu") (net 2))
 (segment (start 121 80.0625) (end 120.9375 80) (width 0.6) (layer "F.Cu") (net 1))
 (segment (start 120.9375 80) (end 120.8125 80) (width 0.6) (layer "F.Cu") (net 1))
 (segment (start 120.8125 80) (end 122.95 80) (width 0.6) (layer "F.Cu") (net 1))
 (segment (start 123 80.05) (end 125.25 80.05) (width 0.6) (layer "F.Cu") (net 1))
 (segment (start 125.25 80.05) (end 125.3 80) (width 0.6) (layer "F.Cu") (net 1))
 (segment (start 122.95 80) (end 123 80.05) (width 0.6) (layer "F.Cu") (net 1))
 (segment (start 144.8125 80) (end 150.75 80) (width 0.6) (layer "F.Cu") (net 5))
 (segment (start 115.25 80) (end 118.6875 80) (width 0.6) (layer "F.Cu") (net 9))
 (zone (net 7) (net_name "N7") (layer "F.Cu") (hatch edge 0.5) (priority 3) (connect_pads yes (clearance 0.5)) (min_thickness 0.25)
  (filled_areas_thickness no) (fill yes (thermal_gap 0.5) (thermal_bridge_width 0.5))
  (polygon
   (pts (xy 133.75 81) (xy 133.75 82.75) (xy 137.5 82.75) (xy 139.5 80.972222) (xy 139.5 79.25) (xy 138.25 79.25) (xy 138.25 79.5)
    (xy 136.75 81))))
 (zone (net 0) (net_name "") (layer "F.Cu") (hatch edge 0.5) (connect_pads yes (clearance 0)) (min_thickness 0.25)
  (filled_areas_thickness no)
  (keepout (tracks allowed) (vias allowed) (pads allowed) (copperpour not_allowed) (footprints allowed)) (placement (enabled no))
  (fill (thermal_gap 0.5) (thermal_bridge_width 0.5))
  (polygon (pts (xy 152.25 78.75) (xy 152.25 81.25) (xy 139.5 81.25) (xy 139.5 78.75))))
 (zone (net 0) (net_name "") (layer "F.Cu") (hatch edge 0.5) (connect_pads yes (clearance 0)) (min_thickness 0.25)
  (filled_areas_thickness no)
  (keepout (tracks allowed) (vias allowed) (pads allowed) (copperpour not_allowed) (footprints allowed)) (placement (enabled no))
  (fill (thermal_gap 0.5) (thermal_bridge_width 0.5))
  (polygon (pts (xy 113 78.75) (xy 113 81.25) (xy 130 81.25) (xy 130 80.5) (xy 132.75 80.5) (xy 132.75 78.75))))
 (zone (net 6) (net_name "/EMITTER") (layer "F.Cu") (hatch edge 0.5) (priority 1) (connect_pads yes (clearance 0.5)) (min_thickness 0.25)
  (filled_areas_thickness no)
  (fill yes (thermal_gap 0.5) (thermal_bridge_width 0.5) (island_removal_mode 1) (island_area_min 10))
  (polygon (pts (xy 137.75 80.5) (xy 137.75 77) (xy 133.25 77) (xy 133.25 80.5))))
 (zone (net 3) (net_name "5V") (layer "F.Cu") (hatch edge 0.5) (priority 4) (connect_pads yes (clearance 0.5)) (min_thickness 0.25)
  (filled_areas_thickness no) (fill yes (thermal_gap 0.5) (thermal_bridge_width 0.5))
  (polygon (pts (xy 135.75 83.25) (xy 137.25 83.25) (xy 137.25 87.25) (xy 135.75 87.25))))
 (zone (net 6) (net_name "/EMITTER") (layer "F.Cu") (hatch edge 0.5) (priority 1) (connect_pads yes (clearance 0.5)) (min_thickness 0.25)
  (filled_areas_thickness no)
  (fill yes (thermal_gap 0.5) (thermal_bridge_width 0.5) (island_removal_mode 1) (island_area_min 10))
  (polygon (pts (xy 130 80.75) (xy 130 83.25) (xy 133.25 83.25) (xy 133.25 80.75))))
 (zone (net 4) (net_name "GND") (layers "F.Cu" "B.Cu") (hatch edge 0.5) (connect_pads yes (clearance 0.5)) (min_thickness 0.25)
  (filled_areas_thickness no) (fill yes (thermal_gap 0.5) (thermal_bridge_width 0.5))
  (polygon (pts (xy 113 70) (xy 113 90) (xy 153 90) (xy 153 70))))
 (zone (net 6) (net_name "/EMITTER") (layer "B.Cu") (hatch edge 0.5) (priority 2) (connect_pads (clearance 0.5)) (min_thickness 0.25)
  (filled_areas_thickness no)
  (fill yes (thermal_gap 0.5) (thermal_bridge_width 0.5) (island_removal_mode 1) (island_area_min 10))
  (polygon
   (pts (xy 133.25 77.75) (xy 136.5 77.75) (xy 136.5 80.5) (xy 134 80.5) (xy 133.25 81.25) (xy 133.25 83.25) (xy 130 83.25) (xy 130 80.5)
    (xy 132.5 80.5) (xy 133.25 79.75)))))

